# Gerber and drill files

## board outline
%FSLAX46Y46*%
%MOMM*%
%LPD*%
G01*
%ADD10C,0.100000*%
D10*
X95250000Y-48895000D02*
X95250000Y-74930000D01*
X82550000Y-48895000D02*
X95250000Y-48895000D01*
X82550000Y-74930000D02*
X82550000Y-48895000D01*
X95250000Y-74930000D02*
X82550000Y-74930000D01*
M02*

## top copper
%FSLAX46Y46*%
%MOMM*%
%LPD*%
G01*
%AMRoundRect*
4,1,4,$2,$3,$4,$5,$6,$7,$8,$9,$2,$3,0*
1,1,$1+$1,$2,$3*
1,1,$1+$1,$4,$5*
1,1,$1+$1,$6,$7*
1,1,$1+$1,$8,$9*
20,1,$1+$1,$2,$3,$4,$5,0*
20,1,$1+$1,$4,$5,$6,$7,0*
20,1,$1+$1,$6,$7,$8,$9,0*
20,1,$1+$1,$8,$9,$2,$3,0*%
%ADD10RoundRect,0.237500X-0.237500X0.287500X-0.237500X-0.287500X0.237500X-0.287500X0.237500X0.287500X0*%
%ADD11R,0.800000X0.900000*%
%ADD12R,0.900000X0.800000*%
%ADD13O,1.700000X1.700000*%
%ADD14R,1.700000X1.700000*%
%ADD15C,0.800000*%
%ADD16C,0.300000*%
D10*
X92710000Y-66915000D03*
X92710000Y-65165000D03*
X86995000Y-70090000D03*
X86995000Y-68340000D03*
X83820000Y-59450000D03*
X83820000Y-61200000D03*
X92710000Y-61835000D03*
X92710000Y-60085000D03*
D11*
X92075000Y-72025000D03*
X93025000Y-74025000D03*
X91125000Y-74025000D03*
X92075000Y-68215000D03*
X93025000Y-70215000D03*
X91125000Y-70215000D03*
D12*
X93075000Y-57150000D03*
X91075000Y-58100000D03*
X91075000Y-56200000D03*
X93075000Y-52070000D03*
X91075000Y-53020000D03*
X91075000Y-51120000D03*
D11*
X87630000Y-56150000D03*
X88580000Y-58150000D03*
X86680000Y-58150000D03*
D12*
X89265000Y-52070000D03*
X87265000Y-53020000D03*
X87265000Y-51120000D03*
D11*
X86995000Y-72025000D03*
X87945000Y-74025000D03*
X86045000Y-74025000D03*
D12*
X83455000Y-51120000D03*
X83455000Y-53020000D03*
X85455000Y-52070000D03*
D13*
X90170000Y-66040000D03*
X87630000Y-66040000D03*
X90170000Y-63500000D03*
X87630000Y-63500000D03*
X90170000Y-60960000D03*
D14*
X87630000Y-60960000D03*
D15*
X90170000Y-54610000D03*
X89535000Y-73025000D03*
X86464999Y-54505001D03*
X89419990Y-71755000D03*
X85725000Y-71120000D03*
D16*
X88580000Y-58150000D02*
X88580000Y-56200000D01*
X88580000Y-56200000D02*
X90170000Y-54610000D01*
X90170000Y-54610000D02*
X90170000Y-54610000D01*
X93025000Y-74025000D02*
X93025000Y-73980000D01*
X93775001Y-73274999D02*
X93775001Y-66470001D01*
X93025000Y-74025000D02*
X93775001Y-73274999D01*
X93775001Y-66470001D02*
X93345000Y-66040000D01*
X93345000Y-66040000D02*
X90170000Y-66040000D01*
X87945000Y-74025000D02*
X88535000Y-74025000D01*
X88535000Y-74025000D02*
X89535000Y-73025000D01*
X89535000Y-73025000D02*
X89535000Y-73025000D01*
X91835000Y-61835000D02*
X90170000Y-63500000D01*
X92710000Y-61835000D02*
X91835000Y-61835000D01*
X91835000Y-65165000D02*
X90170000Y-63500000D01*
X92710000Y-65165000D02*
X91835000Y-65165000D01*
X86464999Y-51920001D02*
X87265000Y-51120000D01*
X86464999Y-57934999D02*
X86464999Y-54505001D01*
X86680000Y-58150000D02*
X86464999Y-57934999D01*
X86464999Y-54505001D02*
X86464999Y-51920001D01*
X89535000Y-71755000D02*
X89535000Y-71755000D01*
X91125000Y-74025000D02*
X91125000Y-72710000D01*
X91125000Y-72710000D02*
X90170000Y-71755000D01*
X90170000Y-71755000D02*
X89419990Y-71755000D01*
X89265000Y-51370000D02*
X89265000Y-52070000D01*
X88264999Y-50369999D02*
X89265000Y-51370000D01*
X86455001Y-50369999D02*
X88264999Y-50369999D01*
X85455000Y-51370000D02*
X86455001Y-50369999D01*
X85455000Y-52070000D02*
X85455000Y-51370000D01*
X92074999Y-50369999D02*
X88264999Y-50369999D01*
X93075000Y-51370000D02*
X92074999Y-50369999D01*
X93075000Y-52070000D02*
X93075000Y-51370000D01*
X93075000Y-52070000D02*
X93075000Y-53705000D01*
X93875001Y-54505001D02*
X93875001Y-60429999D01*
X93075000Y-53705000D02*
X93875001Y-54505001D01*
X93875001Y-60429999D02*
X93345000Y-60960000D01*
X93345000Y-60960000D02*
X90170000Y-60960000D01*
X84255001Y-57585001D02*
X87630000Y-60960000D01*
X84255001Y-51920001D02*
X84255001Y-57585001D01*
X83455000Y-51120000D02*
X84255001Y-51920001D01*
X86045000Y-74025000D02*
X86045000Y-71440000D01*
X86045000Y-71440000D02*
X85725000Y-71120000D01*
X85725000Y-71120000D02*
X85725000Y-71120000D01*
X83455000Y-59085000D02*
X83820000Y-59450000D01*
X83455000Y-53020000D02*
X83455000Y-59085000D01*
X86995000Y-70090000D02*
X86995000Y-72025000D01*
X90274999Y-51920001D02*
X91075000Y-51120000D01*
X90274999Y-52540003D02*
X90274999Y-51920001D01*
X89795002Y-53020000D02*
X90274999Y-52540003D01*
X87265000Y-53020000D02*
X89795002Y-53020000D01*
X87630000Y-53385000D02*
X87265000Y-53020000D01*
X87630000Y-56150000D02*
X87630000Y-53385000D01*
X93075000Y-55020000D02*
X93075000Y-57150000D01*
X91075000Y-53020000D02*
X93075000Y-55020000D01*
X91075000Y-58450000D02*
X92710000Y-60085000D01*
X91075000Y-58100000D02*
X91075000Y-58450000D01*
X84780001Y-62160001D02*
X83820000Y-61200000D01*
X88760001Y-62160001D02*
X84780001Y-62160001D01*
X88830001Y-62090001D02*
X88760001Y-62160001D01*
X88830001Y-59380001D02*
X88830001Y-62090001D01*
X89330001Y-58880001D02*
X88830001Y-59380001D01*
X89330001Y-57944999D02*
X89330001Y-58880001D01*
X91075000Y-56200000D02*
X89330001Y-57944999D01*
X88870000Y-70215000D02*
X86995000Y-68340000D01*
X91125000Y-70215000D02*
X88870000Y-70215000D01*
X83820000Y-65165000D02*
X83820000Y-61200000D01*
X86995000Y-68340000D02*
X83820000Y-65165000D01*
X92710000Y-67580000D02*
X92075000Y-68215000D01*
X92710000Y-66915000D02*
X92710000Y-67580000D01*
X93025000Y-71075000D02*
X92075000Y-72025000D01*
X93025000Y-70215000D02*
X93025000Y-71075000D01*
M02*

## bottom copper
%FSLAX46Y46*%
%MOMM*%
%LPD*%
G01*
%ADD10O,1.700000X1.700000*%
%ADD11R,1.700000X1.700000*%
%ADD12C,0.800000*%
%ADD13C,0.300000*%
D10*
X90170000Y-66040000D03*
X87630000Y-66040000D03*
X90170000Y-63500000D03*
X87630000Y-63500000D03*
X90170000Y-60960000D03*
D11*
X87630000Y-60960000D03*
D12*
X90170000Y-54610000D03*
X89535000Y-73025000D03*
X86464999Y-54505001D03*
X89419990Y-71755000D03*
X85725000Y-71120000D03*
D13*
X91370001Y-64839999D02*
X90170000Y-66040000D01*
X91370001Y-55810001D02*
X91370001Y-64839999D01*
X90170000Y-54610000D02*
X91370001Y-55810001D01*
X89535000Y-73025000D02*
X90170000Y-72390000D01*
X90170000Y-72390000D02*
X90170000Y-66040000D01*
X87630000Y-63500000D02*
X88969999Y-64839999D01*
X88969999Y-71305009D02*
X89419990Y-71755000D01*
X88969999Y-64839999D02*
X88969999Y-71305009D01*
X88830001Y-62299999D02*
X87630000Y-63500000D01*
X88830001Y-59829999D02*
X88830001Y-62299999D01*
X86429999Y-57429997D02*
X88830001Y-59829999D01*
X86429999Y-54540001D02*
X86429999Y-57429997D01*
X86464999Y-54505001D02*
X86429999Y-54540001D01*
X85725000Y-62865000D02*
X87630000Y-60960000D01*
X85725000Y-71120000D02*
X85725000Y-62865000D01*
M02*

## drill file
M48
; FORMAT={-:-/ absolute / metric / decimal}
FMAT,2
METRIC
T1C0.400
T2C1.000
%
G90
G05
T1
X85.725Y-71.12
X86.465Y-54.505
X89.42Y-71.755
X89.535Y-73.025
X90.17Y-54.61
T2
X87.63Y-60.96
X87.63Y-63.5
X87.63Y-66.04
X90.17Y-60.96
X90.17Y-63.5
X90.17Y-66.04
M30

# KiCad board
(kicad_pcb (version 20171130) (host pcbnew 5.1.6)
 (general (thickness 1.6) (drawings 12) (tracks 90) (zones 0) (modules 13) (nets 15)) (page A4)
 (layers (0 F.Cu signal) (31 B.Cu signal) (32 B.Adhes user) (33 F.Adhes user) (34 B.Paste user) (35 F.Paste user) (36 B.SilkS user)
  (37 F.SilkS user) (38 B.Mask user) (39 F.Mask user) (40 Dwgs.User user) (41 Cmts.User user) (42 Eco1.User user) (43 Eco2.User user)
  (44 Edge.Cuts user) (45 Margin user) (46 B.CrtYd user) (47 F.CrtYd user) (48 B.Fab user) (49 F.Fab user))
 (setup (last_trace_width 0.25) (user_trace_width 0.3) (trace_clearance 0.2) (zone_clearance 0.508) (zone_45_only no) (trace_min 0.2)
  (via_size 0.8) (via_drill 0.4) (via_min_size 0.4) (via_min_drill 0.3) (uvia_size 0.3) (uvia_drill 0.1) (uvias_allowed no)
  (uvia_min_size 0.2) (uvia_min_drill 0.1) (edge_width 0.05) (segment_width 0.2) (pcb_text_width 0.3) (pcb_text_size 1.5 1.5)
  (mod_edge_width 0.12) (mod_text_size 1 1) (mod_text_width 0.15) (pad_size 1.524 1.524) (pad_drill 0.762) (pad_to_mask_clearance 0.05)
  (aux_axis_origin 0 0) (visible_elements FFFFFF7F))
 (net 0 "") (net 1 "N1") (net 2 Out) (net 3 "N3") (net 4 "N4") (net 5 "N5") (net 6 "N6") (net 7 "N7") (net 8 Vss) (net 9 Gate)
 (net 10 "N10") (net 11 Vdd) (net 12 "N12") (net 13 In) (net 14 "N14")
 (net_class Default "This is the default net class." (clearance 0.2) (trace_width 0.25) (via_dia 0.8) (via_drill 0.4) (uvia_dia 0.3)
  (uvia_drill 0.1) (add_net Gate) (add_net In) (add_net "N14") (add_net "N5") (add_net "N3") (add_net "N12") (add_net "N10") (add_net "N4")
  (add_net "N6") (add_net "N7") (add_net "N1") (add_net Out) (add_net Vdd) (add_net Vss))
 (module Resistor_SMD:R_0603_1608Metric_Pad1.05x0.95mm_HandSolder (layer F.Cu) (at 92.71 66.04 270)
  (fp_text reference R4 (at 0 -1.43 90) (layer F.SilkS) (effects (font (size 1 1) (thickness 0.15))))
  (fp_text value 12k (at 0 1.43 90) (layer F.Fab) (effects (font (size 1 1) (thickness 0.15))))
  (pad 2 smd roundrect (at 0.875 0 270) (size 1.05 0.95) (layers F.Cu F.Paste F.Mask) (roundrect_rratio 0.25) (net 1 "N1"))
  (pad 1 smd roundrect (at -0.875 0 270) (size 1.05 0.95) (layers F.Cu F.Paste F.Mask) (roundrect_rratio 0.25) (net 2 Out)))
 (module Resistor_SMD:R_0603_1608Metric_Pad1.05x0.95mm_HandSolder (layer F.Cu) (at 86.995 69.215 270)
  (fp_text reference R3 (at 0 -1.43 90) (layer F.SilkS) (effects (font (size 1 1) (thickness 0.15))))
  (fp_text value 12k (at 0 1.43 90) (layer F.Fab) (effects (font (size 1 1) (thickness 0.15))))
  (pad 2 smd roundrect (at 0.875 0 270) (size 1.05 0.95) (layers F.Cu F.Paste F.Mask) (roundrect_rratio 0.25) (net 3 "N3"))
  (pad 1 smd roundrect (at -0.875 0 270) (size 1.05 0.95) (layers F.Cu F.Paste F.Mask) (roundrect_rratio 0.25) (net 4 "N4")))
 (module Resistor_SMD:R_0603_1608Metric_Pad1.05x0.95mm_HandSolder (layer F.Cu) (at 83.82 60.325 270)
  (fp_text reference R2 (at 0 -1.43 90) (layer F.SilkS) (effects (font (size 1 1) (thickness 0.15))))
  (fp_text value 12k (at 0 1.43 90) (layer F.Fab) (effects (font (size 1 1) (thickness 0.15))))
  (pad 1 smd roundrect (at -0.875 0 270) (size 1.05 0.95) (layers F.Cu F.Paste F.Mask) (roundrect_rratio 0.25) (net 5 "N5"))
  (pad 2 smd roundrect (at 0.875 0 270) (size 1.05 0.95) (layers F.Cu F.Paste F.Mask) (roundrect_rratio 0.25) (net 4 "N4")))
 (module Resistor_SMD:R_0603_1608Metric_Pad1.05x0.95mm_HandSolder (layer F.Cu) (at 92.71 60.96 270)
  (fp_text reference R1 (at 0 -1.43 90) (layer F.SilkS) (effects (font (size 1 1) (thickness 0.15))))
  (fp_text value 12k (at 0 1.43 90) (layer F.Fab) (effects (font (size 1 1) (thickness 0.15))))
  (pad 2 smd roundrect (at 0.875 0 270) (size 1.05 0.95) (layers F.Cu F.Paste F.Mask) (roundrect_rratio 0.25) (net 2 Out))
  (pad 1 smd roundrect (at -0.875 0 270) (size 1.05 0.95) (layers F.Cu F.Paste F.Mask) (roundrect_rratio 0.25) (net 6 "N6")))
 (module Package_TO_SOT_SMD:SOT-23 (layer F.Cu) (at 92.075 73.025 90)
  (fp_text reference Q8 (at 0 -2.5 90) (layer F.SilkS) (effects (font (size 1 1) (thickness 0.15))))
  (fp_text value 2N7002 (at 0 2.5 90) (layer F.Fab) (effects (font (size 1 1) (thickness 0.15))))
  (pad 3 smd rect (at 1 0 90) (size 0.9 0.8) (layers F.Cu F.Paste F.Mask) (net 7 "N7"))
  (pad 2 smd rect (at -1 0.95 90) (size 0.9 0.8) (layers F.Cu F.Paste F.Mask) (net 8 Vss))
  (pad 1 smd rect (at -1 -0.95 90) (size 0.9 0.8) (layers F.Cu F.Paste F.Mask) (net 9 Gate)))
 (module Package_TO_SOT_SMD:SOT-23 (layer F.Cu) (at 92.075 69.215 90)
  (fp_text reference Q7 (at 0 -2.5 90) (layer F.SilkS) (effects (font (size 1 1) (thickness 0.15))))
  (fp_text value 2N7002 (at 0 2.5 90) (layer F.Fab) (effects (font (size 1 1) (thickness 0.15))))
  (pad 3 smd rect (at 1 0 90) (size 0.9 0.8) (layers F.Cu F.Paste F.Mask) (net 1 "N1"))
  (pad 2 smd rect (at -1 0.95 90) (size 0.9 0.8) (layers F.Cu F.Paste F.Mask) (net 7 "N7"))
  (pad 1 smd rect (at -1 -0.95 90) (size 0.9 0.8) (layers F.Cu F.Paste F.Mask) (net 4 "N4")))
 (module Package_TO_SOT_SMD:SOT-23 (layer F.Cu) (at 92.075 57.15)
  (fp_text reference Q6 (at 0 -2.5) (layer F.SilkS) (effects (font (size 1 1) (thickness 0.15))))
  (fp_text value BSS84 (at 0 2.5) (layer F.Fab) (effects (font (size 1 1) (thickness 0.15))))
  (pad 3 smd rect (at 1 0) (size 0.9 0.8) (layers F.Cu F.Paste F.Mask) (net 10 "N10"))
  (pad 2 smd rect (at -1 0.95) (size 0.9 0.8) (layers F.Cu F.Paste F.Mask) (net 6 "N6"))
  (pad 1 smd rect (at -1 -0.95) (size 0.9 0.8) (layers F.Cu F.Paste F.Mask) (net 4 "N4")))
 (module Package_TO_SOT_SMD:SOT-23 (layer F.Cu) (at 92.075 52.07)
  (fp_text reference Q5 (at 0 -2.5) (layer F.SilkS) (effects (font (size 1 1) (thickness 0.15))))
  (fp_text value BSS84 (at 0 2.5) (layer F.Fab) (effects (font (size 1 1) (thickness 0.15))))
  (pad 3 smd rect (at 1 0) (size 0.9 0.8) (layers F.Cu F.Paste F.Mask) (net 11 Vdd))
  (pad 2 smd rect (at -1 0.95) (size 0.9 0.8) (layers F.Cu F.Paste F.Mask) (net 10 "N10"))
  (pad 1 smd rect (at -1 -0.95) (size 0.9 0.8) (layers F.Cu F.Paste F.Mask) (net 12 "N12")))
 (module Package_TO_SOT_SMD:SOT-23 (layer F.Cu) (at 87.63 57.15 90)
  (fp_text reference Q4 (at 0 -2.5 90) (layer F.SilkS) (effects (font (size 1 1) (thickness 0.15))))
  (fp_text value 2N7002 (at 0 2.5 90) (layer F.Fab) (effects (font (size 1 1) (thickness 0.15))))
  (pad 3 smd rect (at 1 0 90) (size 0.9 0.8) (layers F.Cu F.Paste F.Mask) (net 12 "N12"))
  (pad 2 smd rect (at -1 0.95 90) (size 0.9 0.8) (layers F.Cu F.Paste F.Mask) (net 8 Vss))
  (pad 1 smd rect (at -1 -0.95 90) (size 0.9 0.8) (layers F.Cu F.Paste F.Mask) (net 9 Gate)))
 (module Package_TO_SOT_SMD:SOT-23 (layer F.Cu) (at 88.265 52.07)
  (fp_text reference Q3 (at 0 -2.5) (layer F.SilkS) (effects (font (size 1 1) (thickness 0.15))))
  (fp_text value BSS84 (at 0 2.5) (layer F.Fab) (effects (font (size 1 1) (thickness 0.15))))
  (pad 3 smd rect (at 1 0) (size 0.9 0.8) (layers F.Cu F.Paste F.Mask) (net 11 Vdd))
  (pad 2 smd rect (at -1 0.95) (size 0.9 0.8) (layers F.Cu F.Paste F.Mask) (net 12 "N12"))
  (pad 1 smd rect (at -1 -0.95) (size 0.9 0.8) (layers F.Cu F.Paste F.Mask) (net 9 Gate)))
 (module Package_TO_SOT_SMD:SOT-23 (layer F.Cu) (at 86.995 73.025 90)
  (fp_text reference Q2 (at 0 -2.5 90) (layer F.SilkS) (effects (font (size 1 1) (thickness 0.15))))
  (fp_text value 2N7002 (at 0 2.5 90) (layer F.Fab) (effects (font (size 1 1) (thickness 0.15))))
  (pad 3 smd rect (at 1 0 90) (size 0.9 0.8) (layers F.Cu F.Paste F.Mask) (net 3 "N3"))
  (pad 2 smd rect (at -1 0.95 90) (size 0.9 0.8) (layers F.Cu F.Paste F.Mask) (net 8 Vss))
  (pad 1 smd rect (at -1 -0.95 90) (size 0.9 0.8) (layers F.Cu F.Paste F.Mask) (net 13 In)))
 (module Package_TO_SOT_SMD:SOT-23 (layer F.Cu) (at 84.455 52.07)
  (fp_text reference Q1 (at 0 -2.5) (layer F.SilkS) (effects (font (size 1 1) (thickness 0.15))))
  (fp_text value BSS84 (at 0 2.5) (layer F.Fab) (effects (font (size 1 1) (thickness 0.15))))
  (pad 1 smd rect (at -1 -0.95) (size 0.9 0.8) (layers F.Cu F.Paste F.Mask) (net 13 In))
  (pad 2 smd rect (at -1 0.95) (size 0.9 0.8) (layers F.Cu F.Paste F.Mask) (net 5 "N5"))
  (pad 3 smd rect (at 1 0) (size 0.9 0.8) (layers F.Cu F.Paste F.Mask) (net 11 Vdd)))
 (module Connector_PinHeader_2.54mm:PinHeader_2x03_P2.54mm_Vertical (layer F.Cu) (at 87.63 60.96)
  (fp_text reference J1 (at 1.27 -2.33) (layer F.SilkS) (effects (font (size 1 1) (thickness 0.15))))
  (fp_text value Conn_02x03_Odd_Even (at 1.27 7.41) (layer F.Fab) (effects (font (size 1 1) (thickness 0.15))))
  (pad 6 thru_hole oval (at 2.54 5.08) (size 1.7 1.7) (drill 1) (layers *.Cu *.Mask) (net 8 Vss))
  (pad 5 thru_hole oval (at 0 5.08) (size 1.7 1.7) (drill 1) (layers *.Cu *.Mask) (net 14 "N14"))
  (pad 4 thru_hole oval (at 2.54 2.54) (size 1.7 1.7) (drill 1) (layers *.Cu *.Mask) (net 2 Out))
  (pad 3 thru_hole oval (at 0 2.54) (size 1.7 1.7) (drill 1) (layers *.Cu *.Mask) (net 9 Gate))
  (pad 2 thru_hole oval (at 2.54 0) (size 1.7 1.7) (drill 1) (layers *.Cu *.Mask) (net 11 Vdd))
  (pad 1 thru_hole rect (at 0 0) (size 1.7 1.7) (drill 1) (layers *.Cu *.Mask) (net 13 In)))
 (gr_line (start 95.25 48.895) (end 95.25 74.93) (layer Edge.Cuts) (width 0.1))
 (gr_line (start 82.55 48.895) (end 95.25 48.895) (layer Edge.Cuts) (width 0.1))
 (gr_line (start 82.55 74.93) (end 82.55 48.895) (layer Edge.Cuts) (width 0.1))
 (gr_line (start 95.25 74.93) (end 82.55 74.93) (layer Edge.Cuts) (width 0.1))
 (segment (start 88.58 58.15) (end 88.58 56.2) (width 0.3) (layer F.Cu) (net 8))
 (segment (start 88.58 56.2) (end 90.17 54.61) (width 0.3) (layer F.Cu) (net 8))
 (segment (start 90.17 54.61) (end 90.17 54.61) (width 0.3) (layer F.Cu) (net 8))
 (via (at 90.17 54.61) (size 0.8) (drill 0.4) (layers F.Cu B.Cu) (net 8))
 (segment (start 93.025 74.025) (end 93.025 73.98) (width 0.3) (layer F.Cu) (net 8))
 (segment (start 93.775001 73.274999) (end 93.775001 66.470001) (width 0.3) (layer F.Cu) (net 8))
 (segment (start 93.025 74.025) (end 93.775001 73.274999) (width 0.3) (layer F.Cu) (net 8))
 (segment (start 93.775001 66.470001) (end 93.345 66.04) (width 0.3) (layer F.Cu) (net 8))
 (segment (start 93.345 66.04) (end 90.17 66.04) (width 0.3) (layer F.Cu) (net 8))
 (segment (start 87.945 74.025) (end 88.535 74.025) (width 0.3) (layer F.Cu) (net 8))
 (segment (start 88.535 74.025) (end 89.535 73.025) (width 0.3) (layer F.Cu) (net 8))
 (segment (start 89.535 73.025) (end 89.535 73.025) (width 0.3) (layer F.Cu) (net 8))
 (via (at 89.535 73.025) (size 0.8) (drill 0.4) (layers F.Cu B.Cu) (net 8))
 (segment (start 91.370001 64.839999) (end 90.17 66.04) (width 0.3) (layer B.Cu) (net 8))
 (segment (start 91.370001 55.810001) (end 91.370001 64.839999) (width 0.3) (layer B.Cu) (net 8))
 (segment (start 90.17 54.61) (end 91.370001 55.810001) (width 0.3) (layer B.Cu) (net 8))
 (segment (start 89.535 73.025) (end 90.17 72.39) (width 0.3) (layer B.Cu) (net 8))
 (segment (start 90.17 72.39) (end 90.17 66.04) (width 0.3) (layer B.Cu) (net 8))
 (segment (start 91.835 61.835) (end 90.17 63.5) (width 0.3) (layer F.Cu) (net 2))
 (segment (start 92.71 61.835) (end 91.835 61.835) (width 0.3) (layer F.Cu) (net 2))
 (segment (start 91.835 65.165) (end 90.17 63.5) (width 0.3) (layer F.Cu) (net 2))
 (segment (start 92.71 65.165) (end 91.835 65.165) (width 0.3) (layer F.Cu) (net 2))
 (segment (start 86.464999 51.920001) (end 87.265 51.12) (width 0.3) (layer F.Cu) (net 9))
 (segment (start 86.464999 57.934999) (end 86.464999 54.505001) (width 0.3) (layer F.Cu) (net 9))
 (segment (start 86.68 58.15) (end 86.464999 57.934999) (width 0.3) (layer F.Cu) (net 9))
 (segment (start 86.464999 54.505001) (end 86.464999 51.920001) (width 0.3) (layer F.Cu) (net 9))
 (via (at 86.464999 54.505001) (size 0.8) (drill 0.4) (layers F.Cu B.Cu) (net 9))
 (segment (start 89.535 71.755) (end 89.535 71.755) (width 0.3) (layer F.Cu) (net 9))
 (via (at 89.41999 71.755) (size 0.8) (drill 0.4) (layers F.Cu B.Cu) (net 9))
 (segment (start 91.125 74.025) (end 91.125 72.71) (width 0.3) (layer F.Cu) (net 9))
 (segment (start 91.125 72.71) (end 90.17 71.755) (width 0.3) (layer F.Cu) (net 9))
 (segment (start 87.63 63.5) (end 88.969999 64.839999) (width 0.3) (layer B.Cu) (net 9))
 (segment (start 88.969999 71.305009) (end 89.41999 71.755) (width 0.3) (layer B.Cu) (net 9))
 (segment (start 88.969999 64.839999) (end 88.969999 71.305009) (width 0.3) (layer B.Cu) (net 9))
 (segment (start 90.17 71.755) (end 89.41999 71.755) (width 0.3) (layer F.Cu) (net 9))
 (segment (start 88.830001 62.299999) (end 87.63 63.5) (width 0.3) (layer B.Cu) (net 9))
 (segment (start 88.830001 59.829999) (end 88.830001 62.299999) (width 0.3) (layer B.Cu) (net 9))
 (segment (start 86.429999 57.429997) (end 88.830001 59.829999) (width 0.3) (layer B.Cu) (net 9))
 (segment (start 86.429999 54.540001) (end 86.429999 57.429997) (width 0.3) (layer B.Cu) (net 9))
 (segment (start 86.464999 54.505001) (end 86.429999 54.540001) (width 0.3) (layer B.Cu) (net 9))
 (segment (start 89.265 51.37) (end 89.265 52.07) (width 0.3) (layer F.Cu) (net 11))
 (segment (start 88.264999 50.369999) (end 89.265 51.37) (width 0.3) (layer F.Cu) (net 11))
 (segment (start 86.455001 50.369999) (end 88.264999 50.369999) (width 0.3) (layer F.Cu) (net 11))
 (segment (start 85.455 51.37) (end 86.455001 50.369999) (width 0.3) (layer F.Cu) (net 11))
 (segment (start 85.455 52.07) (end 85.455 51.37) (width 0.3) (layer F.Cu) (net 11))
 (segment (start 92.074999 50.369999) (end 88.264999 50.369999) (width 0.3) (layer F.Cu) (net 11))
 (segment (start 93.075 51.37) (end 92.074999 50.369999) (width 0.3) (layer F.Cu) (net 11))
 (segment (start 93.075 52.07) (end 93.075 51.37) (width 0.3) (layer F.Cu) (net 11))
 (segment (start 93.075 52.07) (end 93.075 53.705) (width 0.3) (layer F.Cu) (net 11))
 (segment (start 93.875001 54.505001) (end 93.875001 60.429999) (width 0.3) (layer F.Cu) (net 11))
 (segment (start 93.075 53.705) (end 93.875001 54.505001) (width 0.3) (layer F.Cu) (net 11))
 (segment (start 93.875001 60.429999) (end 93.345 60.96) (width 0.3) (layer F.Cu) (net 11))
 (segment (start 93.345 60.96) (end 90.17 60.96) (width 0.3) (layer F.Cu) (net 11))
 (segment (start 84.255001 57.585001) (end 87.63 60.96) (width 0.3) (layer F.Cu) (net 13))
 (segment (start 84.255001 51.920001) (end 84.255001 57.585001) (width 0.3) (layer F.Cu) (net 13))
 (segment (start 83.455 51.12) (end 84.255001 51.920001) (width 0.3) (layer F.Cu) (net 13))
 (segment (start 86.045 74.025) (end 86.045 71.44) (width 0.3) (layer F.Cu) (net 13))
 (segment (start 86.045 71.44) (end 85.725 71.12) (width 0.3) (layer F.Cu) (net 13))
 (segment (start 85.725 71.12) (end 85.725 71.12) (width 0.3) (layer F.Cu) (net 13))
 (via (at 85.725 71.12) (size 0.8) (drill 0.4) (layers F.Cu B.Cu) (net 13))
 (segment (start 85.725 62.865) (end 87.63 60.96) (width 0.3) (layer B.Cu) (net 13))
 (segment (start 85.725 71.12) (end 85.725 62.865) (width 0.3) (layer B.Cu) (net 13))
 (segment (start 83.455 59.085) (end 83.82 59.45) (width 0.3) (layer F.Cu) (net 5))
 (segment (start 83.455 53.02) (end 83.455 59.085) (width 0.3) (layer F.Cu) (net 5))
 (segment (start 86.995 70.09) (end 86.995 72.025) (width 0.3) (layer F.Cu) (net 3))
 (segment (start 90.274999 51.920001) (end 91.075 51.12) (width 0.3) (layer F.Cu) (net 12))
 (segment (start 90.274999 52.540003) (end 90.274999 51.920001) (width 0.3) (layer F.Cu) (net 12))
 (segment (start 89.795002 53.02) (end 90.274999 52.540003) (width 0.3) (layer F.Cu) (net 12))
 (segment (start 87.265 53.02) (end 89.795002 53.02) (width 0.3) (layer F.Cu) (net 12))
 (segment (start 87.63 53.385) (end 87.265 53.02) (width 0.3) (layer F.Cu) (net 12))
 (segment (start 87.63 56.15) (end 87.63 53.385) (width 0.3) (layer F.Cu) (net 12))
 (segment (start 93.075 55.02) (end 93.075 57.15) (width 0.3) (layer F.Cu) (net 10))
 (segment (start 91.075 53.02) (end 93.075 55.02) (width 0.3) (layer F.Cu) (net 10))
 (segment (start 91.075 58.45) (end 92.71 60.085) (width 0.3) (layer F.Cu) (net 6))
 (segment (start 91.075 58.1) (end 91.075 58.45) (width 0.3) (layer F.Cu) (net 6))
 (segment (start 84.780001 62.160001) (end 83.82 61.2) (width 0.3) (layer F.Cu) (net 4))
 (segment (start 88.760001 62.160001) (end 84.780001 62.160001) (width 0.3) (layer F.Cu) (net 4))
 (segment (start 88.830001 62.090001) (end 88.760001 62.160001) (width 0.3) (layer F.Cu) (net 4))
 (segment (start 88.830001 59.380001) (end 88.830001 62.090001) (width 0.3) (layer F.Cu) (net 4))
 (segment (start 89.330001 58.880001) (end 88.830001 59.380001) (width 0.3) (layer F.Cu) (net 4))
 (segment (start 89.330001 57.944999) (end 89.330001 58.880001) (width 0.3) (layer F.Cu) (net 4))
 (segment (start 91.075 56.2) (end 89.330001 57.944999) (width 0.3) (layer F.Cu) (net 4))
 (segment (start 88.87 70.215) (end 86.995 68.34) (width 0.3) (layer F.Cu) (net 4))
 (segment (start 91.125 70.215) (end 88.87 70.215) (width 0.3) (layer F.Cu) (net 4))
 (segment (start 83.82 65.165) (end 83.82 61.2) (width 0.3) (layer F.Cu) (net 4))
 (segment (start 86.995 68.34) (end 83.82 65.165) (width 0.3) (layer F.Cu) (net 4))
 (segment (start 92.71 67.58) (end 92.075 68.215) (width 0.3) (layer F.Cu) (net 1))
 (segment (start 92.71 66.915) (end 92.71 67.58) (width 0.3) (layer F.Cu) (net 1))
 (segment (start 93.025 71.075) (end 92.075 72.025) (width 0.3) (layer F.Cu) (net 7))
 (segment (start 93.025 70.215) (end 93.025 71.075) (width 0.3) (layer F.Cu) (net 7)))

